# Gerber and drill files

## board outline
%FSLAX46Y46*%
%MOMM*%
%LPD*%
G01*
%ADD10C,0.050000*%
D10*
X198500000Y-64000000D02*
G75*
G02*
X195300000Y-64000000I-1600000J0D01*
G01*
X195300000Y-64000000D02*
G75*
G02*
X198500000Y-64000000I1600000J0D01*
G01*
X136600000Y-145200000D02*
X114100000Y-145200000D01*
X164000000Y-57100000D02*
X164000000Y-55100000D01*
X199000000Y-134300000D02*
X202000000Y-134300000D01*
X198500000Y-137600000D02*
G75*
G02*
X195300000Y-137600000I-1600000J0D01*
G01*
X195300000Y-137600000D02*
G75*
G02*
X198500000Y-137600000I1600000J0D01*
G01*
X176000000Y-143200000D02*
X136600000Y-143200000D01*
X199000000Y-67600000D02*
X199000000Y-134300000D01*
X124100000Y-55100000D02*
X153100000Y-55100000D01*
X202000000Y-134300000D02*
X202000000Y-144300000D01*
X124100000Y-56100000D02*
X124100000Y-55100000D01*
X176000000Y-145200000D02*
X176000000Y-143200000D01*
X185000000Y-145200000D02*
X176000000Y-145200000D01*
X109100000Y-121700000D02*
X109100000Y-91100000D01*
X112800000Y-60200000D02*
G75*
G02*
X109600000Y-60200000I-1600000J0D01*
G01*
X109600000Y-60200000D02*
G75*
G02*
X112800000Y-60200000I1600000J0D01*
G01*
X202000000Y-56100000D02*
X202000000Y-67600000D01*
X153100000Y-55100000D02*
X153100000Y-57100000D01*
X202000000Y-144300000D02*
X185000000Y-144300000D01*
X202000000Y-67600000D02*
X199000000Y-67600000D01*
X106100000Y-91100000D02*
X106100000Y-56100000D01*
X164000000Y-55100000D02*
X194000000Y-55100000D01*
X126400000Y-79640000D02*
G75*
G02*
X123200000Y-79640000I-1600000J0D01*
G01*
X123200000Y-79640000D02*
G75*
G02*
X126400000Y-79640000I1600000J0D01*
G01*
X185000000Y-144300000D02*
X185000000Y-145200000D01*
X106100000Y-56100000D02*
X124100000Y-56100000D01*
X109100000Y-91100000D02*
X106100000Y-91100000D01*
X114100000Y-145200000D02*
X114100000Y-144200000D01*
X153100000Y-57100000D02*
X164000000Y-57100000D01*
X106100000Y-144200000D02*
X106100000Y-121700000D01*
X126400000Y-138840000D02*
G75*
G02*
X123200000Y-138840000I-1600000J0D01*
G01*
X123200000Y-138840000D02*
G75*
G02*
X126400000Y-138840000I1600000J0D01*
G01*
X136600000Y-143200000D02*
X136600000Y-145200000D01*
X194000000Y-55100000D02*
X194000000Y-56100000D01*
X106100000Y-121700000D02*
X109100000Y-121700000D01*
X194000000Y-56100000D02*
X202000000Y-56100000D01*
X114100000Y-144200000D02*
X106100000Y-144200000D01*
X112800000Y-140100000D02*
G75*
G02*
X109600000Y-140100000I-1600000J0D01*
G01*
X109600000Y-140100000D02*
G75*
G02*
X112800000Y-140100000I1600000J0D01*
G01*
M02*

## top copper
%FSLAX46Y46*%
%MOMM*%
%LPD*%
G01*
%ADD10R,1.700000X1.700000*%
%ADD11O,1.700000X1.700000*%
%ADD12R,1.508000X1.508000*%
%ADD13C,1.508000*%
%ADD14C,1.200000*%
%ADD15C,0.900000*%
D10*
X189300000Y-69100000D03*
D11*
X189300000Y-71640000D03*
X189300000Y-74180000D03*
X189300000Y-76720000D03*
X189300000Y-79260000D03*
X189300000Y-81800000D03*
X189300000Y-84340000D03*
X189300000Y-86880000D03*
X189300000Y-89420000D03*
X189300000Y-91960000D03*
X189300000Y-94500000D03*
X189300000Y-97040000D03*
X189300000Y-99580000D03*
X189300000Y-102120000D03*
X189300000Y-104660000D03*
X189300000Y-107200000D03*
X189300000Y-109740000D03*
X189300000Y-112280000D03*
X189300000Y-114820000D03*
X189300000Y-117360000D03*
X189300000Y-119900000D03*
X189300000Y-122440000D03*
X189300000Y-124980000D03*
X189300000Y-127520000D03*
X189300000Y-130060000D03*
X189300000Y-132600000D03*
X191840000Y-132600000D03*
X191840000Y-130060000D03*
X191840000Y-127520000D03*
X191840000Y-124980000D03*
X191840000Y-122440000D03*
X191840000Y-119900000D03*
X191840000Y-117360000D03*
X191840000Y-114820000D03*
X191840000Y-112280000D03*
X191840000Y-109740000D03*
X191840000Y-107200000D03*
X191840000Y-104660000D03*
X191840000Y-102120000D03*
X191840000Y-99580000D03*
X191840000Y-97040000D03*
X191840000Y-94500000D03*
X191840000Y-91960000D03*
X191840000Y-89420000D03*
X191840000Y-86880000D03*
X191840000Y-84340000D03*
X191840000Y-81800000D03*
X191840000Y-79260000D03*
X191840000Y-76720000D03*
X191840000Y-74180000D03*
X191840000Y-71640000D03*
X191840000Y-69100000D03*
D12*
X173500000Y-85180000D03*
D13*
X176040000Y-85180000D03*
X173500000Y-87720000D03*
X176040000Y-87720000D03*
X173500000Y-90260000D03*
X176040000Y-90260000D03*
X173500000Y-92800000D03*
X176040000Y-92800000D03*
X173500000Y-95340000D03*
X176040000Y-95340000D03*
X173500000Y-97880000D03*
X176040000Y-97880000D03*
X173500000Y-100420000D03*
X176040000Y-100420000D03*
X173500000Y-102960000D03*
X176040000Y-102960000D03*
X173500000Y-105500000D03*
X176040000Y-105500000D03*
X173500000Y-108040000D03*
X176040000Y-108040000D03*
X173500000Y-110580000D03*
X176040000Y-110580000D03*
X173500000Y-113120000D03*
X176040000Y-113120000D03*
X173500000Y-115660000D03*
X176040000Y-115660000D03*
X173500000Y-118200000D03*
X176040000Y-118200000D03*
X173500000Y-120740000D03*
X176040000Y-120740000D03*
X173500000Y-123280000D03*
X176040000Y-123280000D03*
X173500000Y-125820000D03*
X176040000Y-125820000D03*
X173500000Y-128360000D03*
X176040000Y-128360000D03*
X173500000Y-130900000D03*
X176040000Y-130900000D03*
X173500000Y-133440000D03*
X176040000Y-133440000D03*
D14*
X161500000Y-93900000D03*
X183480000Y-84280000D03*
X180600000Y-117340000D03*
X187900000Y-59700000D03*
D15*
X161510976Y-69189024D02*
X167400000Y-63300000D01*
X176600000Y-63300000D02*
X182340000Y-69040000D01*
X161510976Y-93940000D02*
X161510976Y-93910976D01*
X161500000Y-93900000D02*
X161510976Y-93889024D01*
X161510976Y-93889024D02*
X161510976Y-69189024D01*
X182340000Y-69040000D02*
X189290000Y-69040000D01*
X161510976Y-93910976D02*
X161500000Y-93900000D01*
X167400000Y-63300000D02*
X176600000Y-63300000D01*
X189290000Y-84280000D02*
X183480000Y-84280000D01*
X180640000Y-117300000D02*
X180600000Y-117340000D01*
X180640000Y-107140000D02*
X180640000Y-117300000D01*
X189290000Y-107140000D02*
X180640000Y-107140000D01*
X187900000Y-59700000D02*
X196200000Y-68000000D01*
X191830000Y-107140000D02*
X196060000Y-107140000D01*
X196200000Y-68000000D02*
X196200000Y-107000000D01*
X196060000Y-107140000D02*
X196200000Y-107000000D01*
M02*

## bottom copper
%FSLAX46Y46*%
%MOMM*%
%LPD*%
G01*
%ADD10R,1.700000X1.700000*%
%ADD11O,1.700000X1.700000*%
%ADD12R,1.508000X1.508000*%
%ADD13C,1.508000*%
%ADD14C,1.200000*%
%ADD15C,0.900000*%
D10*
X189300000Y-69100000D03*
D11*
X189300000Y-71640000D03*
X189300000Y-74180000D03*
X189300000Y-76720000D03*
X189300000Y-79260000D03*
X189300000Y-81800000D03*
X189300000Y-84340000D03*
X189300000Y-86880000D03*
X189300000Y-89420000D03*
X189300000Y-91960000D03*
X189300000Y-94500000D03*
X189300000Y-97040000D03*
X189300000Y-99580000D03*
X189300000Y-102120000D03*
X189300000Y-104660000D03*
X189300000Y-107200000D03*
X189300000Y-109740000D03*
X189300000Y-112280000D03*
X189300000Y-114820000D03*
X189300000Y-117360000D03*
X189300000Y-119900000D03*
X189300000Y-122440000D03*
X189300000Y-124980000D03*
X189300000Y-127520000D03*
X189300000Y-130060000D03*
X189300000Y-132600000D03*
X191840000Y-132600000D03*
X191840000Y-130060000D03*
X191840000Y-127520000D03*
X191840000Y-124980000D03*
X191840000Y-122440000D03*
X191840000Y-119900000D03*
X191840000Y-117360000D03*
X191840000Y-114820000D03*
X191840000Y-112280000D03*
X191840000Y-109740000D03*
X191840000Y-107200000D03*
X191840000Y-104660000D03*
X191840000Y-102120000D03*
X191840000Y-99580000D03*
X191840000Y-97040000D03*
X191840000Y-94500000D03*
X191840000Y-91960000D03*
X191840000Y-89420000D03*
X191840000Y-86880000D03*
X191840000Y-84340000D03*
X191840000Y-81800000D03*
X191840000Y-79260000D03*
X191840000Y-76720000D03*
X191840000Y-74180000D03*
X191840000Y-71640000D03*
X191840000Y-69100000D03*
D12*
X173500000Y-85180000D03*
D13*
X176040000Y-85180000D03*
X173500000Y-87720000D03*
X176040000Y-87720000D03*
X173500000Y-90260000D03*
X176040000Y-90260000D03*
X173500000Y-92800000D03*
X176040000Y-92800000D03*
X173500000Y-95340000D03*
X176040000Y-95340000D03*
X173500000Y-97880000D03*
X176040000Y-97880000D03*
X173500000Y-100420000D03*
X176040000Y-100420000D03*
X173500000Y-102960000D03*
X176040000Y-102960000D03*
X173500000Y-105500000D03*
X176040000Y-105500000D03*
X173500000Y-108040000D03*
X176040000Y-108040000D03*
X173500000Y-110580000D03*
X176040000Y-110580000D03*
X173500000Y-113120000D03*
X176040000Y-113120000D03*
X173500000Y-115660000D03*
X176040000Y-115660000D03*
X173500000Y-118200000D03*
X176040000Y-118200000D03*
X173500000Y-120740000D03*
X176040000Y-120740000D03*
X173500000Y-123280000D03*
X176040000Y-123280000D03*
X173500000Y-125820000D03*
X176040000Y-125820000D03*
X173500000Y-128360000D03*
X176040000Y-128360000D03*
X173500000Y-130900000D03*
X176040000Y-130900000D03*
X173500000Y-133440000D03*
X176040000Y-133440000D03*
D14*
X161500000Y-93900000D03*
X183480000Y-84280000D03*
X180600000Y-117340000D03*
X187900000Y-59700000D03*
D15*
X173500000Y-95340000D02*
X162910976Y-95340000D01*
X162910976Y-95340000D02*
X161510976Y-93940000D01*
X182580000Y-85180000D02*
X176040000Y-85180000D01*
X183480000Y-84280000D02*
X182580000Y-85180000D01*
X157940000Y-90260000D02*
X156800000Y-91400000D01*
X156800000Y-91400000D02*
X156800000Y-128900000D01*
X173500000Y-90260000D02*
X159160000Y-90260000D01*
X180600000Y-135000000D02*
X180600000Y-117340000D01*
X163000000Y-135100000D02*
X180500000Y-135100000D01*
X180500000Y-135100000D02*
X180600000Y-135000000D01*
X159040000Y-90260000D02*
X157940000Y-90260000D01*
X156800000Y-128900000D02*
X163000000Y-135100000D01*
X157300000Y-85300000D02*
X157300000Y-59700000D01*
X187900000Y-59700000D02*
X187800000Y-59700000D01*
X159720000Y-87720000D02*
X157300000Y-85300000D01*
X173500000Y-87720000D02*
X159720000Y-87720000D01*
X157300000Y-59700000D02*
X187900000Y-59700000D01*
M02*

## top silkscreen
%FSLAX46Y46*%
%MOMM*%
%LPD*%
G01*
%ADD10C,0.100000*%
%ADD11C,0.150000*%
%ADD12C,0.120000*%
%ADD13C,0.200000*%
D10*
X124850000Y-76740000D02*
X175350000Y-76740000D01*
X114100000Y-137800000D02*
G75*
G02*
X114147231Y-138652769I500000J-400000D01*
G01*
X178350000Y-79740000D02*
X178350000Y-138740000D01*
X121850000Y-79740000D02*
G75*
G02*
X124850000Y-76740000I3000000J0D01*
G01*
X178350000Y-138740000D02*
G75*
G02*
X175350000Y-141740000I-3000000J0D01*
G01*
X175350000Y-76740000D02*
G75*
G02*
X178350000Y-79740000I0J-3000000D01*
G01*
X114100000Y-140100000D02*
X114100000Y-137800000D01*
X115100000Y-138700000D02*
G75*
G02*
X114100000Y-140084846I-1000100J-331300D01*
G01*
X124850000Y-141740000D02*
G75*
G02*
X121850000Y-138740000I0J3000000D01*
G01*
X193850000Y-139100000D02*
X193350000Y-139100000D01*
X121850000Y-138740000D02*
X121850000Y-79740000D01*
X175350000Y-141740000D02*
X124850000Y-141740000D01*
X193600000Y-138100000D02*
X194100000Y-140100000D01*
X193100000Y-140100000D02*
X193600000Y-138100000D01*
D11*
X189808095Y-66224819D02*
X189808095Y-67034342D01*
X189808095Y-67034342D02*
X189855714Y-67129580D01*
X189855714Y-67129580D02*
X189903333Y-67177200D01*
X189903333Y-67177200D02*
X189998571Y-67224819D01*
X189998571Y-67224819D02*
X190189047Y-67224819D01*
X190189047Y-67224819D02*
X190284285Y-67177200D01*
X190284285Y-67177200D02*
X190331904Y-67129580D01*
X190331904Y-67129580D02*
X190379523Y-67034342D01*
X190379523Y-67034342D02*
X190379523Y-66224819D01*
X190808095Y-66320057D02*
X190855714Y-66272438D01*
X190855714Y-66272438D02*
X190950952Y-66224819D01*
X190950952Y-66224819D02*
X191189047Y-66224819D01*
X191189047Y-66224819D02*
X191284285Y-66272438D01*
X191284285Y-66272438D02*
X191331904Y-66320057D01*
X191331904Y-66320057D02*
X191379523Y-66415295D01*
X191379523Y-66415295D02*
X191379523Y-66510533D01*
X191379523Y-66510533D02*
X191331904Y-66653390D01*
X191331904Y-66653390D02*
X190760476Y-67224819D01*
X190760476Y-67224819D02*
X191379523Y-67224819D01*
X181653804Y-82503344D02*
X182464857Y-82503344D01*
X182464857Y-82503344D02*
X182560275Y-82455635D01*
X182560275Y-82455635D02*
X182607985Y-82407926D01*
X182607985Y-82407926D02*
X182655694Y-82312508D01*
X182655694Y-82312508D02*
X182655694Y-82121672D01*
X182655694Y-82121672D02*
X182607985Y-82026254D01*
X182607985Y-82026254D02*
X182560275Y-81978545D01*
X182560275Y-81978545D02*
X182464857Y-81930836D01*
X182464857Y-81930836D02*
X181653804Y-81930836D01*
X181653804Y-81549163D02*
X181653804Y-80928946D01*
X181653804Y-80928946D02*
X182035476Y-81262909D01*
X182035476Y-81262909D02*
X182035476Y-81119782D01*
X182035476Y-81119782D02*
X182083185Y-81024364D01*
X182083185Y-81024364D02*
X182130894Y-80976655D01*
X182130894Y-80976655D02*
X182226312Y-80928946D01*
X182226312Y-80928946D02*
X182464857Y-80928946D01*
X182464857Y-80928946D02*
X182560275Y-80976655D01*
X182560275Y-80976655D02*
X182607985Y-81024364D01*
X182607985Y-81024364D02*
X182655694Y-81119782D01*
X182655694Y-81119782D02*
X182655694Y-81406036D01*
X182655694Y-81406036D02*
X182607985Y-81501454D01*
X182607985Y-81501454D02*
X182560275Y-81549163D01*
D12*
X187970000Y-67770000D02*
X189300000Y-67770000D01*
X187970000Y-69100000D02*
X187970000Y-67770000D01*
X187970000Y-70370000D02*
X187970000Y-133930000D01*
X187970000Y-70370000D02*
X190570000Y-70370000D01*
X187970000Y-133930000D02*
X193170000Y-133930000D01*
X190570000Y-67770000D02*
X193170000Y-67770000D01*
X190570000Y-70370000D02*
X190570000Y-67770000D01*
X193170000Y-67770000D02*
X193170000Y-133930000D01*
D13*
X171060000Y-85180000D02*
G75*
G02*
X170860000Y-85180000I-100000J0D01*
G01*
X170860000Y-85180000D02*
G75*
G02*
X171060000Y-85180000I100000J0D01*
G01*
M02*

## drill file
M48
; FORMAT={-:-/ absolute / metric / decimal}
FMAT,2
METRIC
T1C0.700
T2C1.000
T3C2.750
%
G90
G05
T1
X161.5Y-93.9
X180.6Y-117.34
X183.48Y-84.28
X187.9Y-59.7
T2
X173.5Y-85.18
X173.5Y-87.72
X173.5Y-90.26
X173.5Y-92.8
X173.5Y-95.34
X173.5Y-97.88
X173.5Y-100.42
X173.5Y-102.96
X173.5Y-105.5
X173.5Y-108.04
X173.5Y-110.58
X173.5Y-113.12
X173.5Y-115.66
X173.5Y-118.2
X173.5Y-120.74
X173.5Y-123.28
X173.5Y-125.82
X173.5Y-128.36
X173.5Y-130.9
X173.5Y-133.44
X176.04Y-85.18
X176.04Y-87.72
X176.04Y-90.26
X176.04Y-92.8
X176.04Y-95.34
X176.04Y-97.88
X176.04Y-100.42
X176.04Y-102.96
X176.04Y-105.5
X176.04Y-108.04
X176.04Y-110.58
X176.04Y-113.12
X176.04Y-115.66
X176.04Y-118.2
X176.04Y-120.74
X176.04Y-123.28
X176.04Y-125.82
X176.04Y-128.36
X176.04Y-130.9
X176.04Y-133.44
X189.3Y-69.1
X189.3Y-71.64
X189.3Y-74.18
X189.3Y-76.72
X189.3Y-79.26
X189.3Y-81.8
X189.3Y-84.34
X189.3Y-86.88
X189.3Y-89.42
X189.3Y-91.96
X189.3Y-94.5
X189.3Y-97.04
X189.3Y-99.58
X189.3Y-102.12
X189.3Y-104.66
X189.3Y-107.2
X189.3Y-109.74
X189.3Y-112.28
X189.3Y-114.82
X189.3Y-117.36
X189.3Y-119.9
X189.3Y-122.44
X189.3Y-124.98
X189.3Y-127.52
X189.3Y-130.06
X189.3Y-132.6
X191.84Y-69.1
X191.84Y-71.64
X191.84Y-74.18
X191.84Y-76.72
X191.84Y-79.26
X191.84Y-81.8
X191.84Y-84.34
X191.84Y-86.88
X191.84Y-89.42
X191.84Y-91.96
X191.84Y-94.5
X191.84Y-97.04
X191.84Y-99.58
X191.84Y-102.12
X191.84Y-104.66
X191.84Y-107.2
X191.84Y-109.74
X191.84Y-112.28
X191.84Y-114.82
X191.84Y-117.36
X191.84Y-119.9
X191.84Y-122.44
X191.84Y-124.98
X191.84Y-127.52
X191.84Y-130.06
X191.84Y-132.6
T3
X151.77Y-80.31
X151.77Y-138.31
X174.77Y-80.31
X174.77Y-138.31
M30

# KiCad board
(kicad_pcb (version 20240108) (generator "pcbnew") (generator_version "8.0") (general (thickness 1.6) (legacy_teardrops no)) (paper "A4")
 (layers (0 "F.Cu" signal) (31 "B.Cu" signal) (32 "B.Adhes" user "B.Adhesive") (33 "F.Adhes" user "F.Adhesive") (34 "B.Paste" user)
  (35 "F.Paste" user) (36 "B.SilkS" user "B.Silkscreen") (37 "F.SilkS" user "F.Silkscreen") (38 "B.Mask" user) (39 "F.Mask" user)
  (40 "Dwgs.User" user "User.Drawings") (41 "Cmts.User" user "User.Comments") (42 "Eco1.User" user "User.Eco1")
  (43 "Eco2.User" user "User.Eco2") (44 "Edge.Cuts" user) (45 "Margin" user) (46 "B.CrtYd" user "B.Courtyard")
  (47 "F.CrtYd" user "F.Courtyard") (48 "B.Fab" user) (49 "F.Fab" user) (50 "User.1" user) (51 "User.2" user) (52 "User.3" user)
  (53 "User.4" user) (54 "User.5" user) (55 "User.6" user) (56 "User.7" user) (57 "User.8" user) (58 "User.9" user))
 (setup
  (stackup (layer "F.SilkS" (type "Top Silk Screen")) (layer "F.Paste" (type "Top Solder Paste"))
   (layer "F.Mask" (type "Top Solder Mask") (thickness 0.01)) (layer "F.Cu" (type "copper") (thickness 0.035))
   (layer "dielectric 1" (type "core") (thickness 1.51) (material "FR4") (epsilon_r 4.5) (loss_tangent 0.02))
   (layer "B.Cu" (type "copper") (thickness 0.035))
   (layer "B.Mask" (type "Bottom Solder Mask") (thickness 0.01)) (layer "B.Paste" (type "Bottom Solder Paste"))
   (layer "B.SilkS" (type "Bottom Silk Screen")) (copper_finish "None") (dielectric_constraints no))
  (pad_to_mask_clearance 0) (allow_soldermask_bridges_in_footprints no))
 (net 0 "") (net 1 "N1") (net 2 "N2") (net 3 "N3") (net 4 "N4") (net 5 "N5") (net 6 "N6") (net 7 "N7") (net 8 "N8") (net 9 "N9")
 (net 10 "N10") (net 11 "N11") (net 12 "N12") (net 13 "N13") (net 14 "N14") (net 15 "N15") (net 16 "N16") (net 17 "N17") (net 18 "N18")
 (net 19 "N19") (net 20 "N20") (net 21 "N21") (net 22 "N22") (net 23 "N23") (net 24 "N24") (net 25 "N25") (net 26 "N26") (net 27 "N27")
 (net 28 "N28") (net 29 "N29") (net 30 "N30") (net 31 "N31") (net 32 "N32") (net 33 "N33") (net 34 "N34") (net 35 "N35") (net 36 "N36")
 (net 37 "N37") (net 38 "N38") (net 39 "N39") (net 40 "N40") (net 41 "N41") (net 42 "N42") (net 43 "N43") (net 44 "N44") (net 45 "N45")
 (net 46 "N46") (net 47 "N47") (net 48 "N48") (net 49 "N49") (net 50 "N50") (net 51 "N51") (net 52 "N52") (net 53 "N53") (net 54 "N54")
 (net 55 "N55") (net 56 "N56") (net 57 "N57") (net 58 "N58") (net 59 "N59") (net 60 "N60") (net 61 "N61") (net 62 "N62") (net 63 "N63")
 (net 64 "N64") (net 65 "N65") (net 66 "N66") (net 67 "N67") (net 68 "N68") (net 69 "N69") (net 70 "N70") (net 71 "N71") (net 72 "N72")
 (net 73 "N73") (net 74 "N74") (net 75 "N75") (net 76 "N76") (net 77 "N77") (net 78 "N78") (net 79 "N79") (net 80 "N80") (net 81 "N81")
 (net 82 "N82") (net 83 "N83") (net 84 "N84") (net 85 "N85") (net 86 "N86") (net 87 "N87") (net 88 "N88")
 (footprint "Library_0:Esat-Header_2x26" (layer "F.Cu") (at 189.3 69.1)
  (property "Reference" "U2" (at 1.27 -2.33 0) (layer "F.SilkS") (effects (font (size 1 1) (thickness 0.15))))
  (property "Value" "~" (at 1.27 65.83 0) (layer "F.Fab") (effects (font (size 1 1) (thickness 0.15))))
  (fp_line (start -1.33 -1.33) (end 0 -1.33) (stroke (width 0.12) (type solid)) (layer "F.SilkS"))
  (fp_line (start -1.33 0) (end -1.33 -1.33) (stroke (width 0.12) (type solid)) (layer "F.SilkS"))
  (fp_line (start -1.33 1.27) (end -1.33 64.83) (stroke (width 0.12) (type solid)) (layer "F.SilkS"))
  (fp_line (start -1.33 1.27) (end 1.27 1.27) (stroke (width 0.12) (type solid)) (layer "F.SilkS"))
  (fp_line (start -1.33 64.83) (end 3.87 64.83) (stroke (width 0.12) (type solid)) (layer "F.SilkS"))
  (fp_line (start 1.27 -1.33) (end 3.87 -1.33) (stroke (width 0.12) (type solid)) (layer "F.SilkS"))
  (fp_line (start 1.27 1.27) (end 1.27 -1.33) (stroke (width 0.12) (type solid)) (layer "F.SilkS"))
  (fp_line (start 3.87 -1.33) (end 3.87 64.83) (stroke (width 0.12) (type solid)) (layer "F.SilkS"))
  (pad "1" thru_hole rect (at 0 0) (size 1.7 1.7) (drill 1) (layers "*.Cu" "*.Mask") (remove_unused_layers no) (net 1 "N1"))
  (pad "2" thru_hole oval (at 0 2.54) (size 1.7 1.7) (drill 1) (layers "*.Cu" "*.Mask" "B.Paste") (remove_unused_layers no) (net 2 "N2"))
  (pad "3" thru_hole oval (at 0 5.08) (size 1.7 1.7) (drill 1) (layers "*.Cu" "*.Mask") (remove_unused_layers no) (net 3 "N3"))
  (pad "4" thru_hole oval (at 0 7.62) (size 1.7 1.7) (drill 1) (layers "*.Cu" "*.Mask") (remove_unused_layers no) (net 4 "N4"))
  (pad "5" thru_hole oval (at 0 10.16) (size 1.7 1.7) (drill 1) (layers "*.Cu" "*.Mask") (remove_unused_layers no) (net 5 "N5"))
  (pad "6" thru_hole oval (at 0 12.7) (size 1.7 1.7) (drill 1) (layers "*.Cu" "*.Mask") (remove_unused_layers no) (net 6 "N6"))
  (pad "7" thru_hole oval (at 0 15.24) (size 1.7 1.7) (drill 1) (layers "*.Cu" "*.Mask") (remove_unused_layers no) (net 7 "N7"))
  (pad "8" thru_hole oval (at 0 17.78) (size 1.7 1.7) (drill 1) (layers "*.Cu" "*.Mask") (remove_unused_layers no) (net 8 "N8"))
  (pad "9" thru_hole oval (at 0 20.32) (size 1.7 1.7) (drill 1) (layers "*.Cu" "*.Mask") (remove_unused_layers no) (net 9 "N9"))
  (pad "10" thru_hole oval (at 0 22.86) (size 1.7 1.7) (drill 1) (layers "*.Cu" "*.Mask") (remove_unused_layers no) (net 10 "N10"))
  (pad "11" thru_hole oval (at 0 25.4) (size 1.7 1.7) (drill 1) (layers "*.Cu" "*.Mask") (remove_unused_layers no) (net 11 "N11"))
  (pad "12" thru_hole oval (at 0 27.94) (size 1.7 1.7) (drill 1) (layers "*.Cu" "*.Mask") (remove_unused_layers no) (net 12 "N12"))
  (pad "13" thru_hole oval (at 0 30.48) (size 1.7 1.7) (drill 1) (layers "*.Cu" "*.Mask") (remove_unused_layers no) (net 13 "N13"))
  (pad "14" thru_hole oval (at 0 33.02) (size 1.7 1.7) (drill 1) (layers "*.Cu" "*.Mask") (remove_unused_layers no) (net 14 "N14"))
  (pad "15" thru_hole oval (at 0 35.56) (size 1.7 1.7) (drill 1) (layers "*.Cu" "*.Mask") (remove_unused_layers no) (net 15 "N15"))
  (pad "16" thru_hole oval (at 0 38.1) (size 1.7 1.7) (drill 1) (layers "*.Cu" "*.Mask") (remove_unused_layers no) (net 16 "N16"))
  (pad "17" thru_hole oval (at 0 40.64) (size 1.7 1.7) (drill 1) (layers "*.Cu" "*.Mask") (remove_unused_layers no) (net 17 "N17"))
  (pad "18" thru_hole oval (at 0 43.18) (size 1.7 1.7) (drill 1) (layers "*.Cu" "*.Mask") (remove_unused_layers no) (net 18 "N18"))
  (pad "19" thru_hole oval (at 0 45.72) (size 1.7 1.7) (drill 1) (layers "*.Cu" "*.Mask") (remove_unused_layers no) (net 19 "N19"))
  (pad "20" thru_hole oval (at 0 48.26) (size 1.7 1.7) (drill 1) (layers "*.Cu" "*.Mask") (remove_unused_layers no) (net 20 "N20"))
  (pad "21" thru_hole oval (at 0 50.8) (size 1.7 1.7) (drill 1) (layers "*.Cu" "B.Mask") (remove_unused_layers no) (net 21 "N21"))
  (pad "22" thru_hole oval (at 0 53.34) (size 1.7 1.7) (drill 1) (layers "*.Cu" "*.Mask") (remove_unused_layers no) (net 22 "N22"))
  (pad "23" thru_hole oval (at 0 55.88) (size 1.7 1.7) (drill 1) (layers "*.Cu" "*.Mask") (remove_unused_layers no) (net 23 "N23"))
  (pad "24" thru_hole oval (at 0 58.42) (size 1.7 1.7) (drill 1) (layers "*.Cu" "*.Mask") (remove_unused_layers no) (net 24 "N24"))
  (pad "25" thru_hole oval (at 0 60.96) (size 1.7 1.7) (drill 1) (layers "*.Cu" "*.Mask") (remove_unused_layers no) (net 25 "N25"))
  (pad "26" thru_hole oval (at 0 63.5) (size 1.7 1.7) (drill 1) (layers "*.Cu" "*.Mask") (remove_unused_layers no) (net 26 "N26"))
  (pad "27" thru_hole oval (at 2.54 63.5) (size 1.7 1.7) (drill 1) (layers "*.Cu" "*.Mask") (remove_unused_layers no) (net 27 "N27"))
  (pad "28" thru_hole oval (at 2.54 60.96) (size 1.7 1.7) (drill 1) (layers "*.Cu" "*.Mask") (remove_unused_layers no) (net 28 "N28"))
  (pad "29" thru_hole oval (at 2.54 58.42) (size 1.7 1.7) (drill 1) (layers "*.Cu" "*.Mask") (remove_unused_layers no) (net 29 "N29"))
  (pad "30" thru_hole oval (at 2.54 55.88) (size 1.7 1.7) (drill 1) (layers "*.Cu" "*.Mask") (remove_unused_layers no) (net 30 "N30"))
  (pad "31" thru_hole oval (at 2.54 53.34) (size 1.7 1.7) (drill 1) (layers "*.Cu" "*.Mask") (remove_unused_layers no) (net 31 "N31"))
  (pad "32" thru_hole oval (at 2.54 50.8) (size 1.7 1.7) (drill 1) (layers "*.Cu" "*.Mask") (remove_unused_layers no) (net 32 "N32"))
  (pad "33" thru_hole oval (at 2.54 48.26) (size 1.7 1.7) (drill 1) (layers "*.Cu" "*.Mask") (remove_unused_layers no) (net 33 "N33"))
  (pad "34" thru_hole oval (at 2.54 45.72) (size 1.7 1.7) (drill 1) (layers "*.Cu" "*.Mask") (remove_unused_layers no) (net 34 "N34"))
  (pad "35" thru_hole oval (at 2.54 43.18) (size 1.7 1.7) (drill 1) (layers "*.Cu" "*.Mask") (remove_unused_layers no) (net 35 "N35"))
  (pad "36" thru_hole oval (at 2.54 40.64) (size 1.7 1.7) (drill 1) (layers "*.Cu" "*.Mask") (remove_unused_layers no) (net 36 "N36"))
  (pad "37" thru_hole oval (at 2.54 38.1) (size 1.7 1.7) (drill 1) (layers "*.Cu" "*.Mask") (remove_unused_layers no) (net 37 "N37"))
  (pad "38" thru_hole oval (at 2.54 35.56) (size 1.7 1.7) (drill 1) (layers "*.Cu" "*.Mask") (remove_unused_layers no) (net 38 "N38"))
  (pad "39" thru_hole oval (at 2.54 33.02) (size 1.7 1.7) (drill 1) (layers "*.Cu" "*.Mask" "B.Adhes") (remove_unused_layers no)
   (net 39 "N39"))
  (pad "40" thru_hole oval (at 2.54 30.48) (size 1.7 1.7) (drill 1) (layers "*.Cu" "*.Mask") (remove_unused_layers no) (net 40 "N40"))
  (pad "41" thru_hole oval (at 2.54 27.94) (size 1.7 1.7) (drill 1) (layers "*.Cu" "*.Mask") (remove_unused_layers no) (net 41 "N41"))
  (pad "42" thru_hole oval (at 2.54 25.4) (size 1.7 1.7) (drill 1) (layers "*.Cu" "*.Mask") (remove_unused_layers no) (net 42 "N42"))
  (pad "43" thru_hole oval (at 2.54 22.86) (size 1.7 1.7) (drill 1) (layers "*.Cu" "*.Mask") (remove_unused_layers no) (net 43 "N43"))
  (pad "44" thru_hole oval (at 2.54 20.32) (size 1.7 1.7) (drill 1) (layers "*.Cu" "*.Mask") (remove_unused_layers no) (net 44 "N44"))
  (pad "45" thru_hole oval (at 2.54 17.78) (size 1.7 1.7) (drill 1) (layers "*.Cu" "*.Mask") (remove_unused_layers no) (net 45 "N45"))
  (pad "46" thru_hole oval (at 2.54 15.24) (size 1.7 1.7) (drill 1) (layers "*.Cu" "*.Mask") (remove_unused_layers no) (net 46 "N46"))
  (pad "47" thru_hole oval (at 2.54 12.7) (size 1.7 1.7) (drill 1) (layers "*.Cu" "*.Mask") (remove_unused_layers no) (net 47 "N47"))
  (pad "48" thru_hole oval (at 2.54 10.16) (size 1.7 1.7) (drill 1) (layers "*.Cu" "*.Mask") (remove_unused_layers no) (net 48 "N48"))
  (pad "49" thru_hole oval (at 2.54 7.62) (size 1.7 1.7) (drill 1) (layers "*.Cu" "*.Mask") (remove_unused_layers no) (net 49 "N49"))
  (pad "50" thru_hole oval (at 2.54 5.08) (size 1.7 1.7) (drill 1) (layers "*.Cu" "*.Mask") (remove_unused_layers no) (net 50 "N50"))
  (pad "51" thru_hole oval (at 2.54 2.54) (size 1.7 1.7) (drill 1) (layers "*.Cu" "*.Mask") (remove_unused_layers no) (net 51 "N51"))
  (pad "52" thru_hole oval (at 2.54 0) (size 1.7 1.7) (drill 1) (layers "*.Cu" "*.Mask") (remove_unused_layers no) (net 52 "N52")))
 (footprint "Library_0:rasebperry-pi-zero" (layer "F.Cu") (at 163.27 109.31 -90)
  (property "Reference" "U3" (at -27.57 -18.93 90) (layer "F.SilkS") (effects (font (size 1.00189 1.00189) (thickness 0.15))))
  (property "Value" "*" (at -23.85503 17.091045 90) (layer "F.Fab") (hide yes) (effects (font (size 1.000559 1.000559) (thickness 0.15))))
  (fp_circle (center -24.13 -7.69) (end -24.03 -7.69) (stroke (width 0.2) (type solid)) (fill none) (layer "F.SilkS"))
  (pad "" np_thru_hole circle (at -29 -11.5 270) (size 2.75 2.75) (drill 2.75) (layers "*.Cu" "*.Mask"))
  (pad "" np_thru_hole circle (at -29 11.5 270) (size 2.75 2.75) (drill 2.75) (layers "*.Cu" "*.Mask"))
  (pad "" np_thru_hole circle (at 29 -11.5 270) (size 2.75 2.75) (drill 2.75) (layers "*.Cu" "*.Mask"))
  (pad "" np_thru_hole circle (at 29 11.5 270) (size 2.75 2.75) (drill 2.75) (layers "*.Cu" "*.Mask"))
  (pad "1" thru_hole rect (at -24.13 -10.23 270) (size 1.508 1.508) (drill 1) (layers "*.Cu" "*.Mask") (remove_unused_layers no)
   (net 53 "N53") (solder_mask_margin 0.102))
  (pad "2" thru_hole circle (at -24.13 -12.77 270) (size 1.508 1.508) (drill 1) (layers "*.Cu" "*.Mask") (remove_unused_layers no)
   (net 7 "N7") (solder_mask_margin 0.102))
  (pad "3" thru_hole circle (at -21.59 -10.23 270) (size 1.508 1.508) (drill 1) (layers "*.Cu" "*.Mask") (remove_unused_layers no)
   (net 37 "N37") (solder_mask_margin 0.102))
  (pad "4" thru_hole circle (at -21.59 -12.77 270) (size 1.508 1.508) (drill 1) (layers "*.Cu" "*.Mask") (remove_unused_layers no)
   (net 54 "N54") (solder_mask_margin 0.102))
  (pad "5" thru_hole circle (at -19.05 -10.23 270) (size 1.508 1.508) (drill 1) (layers "*.Cu" "*.Mask") (remove_unused_layers no)
   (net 16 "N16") (solder_mask_margin 0.102))
  (pad "6" thru_hole circle (at -19.05 -12.77 270) (size 1.508 1.508) (drill 1) (layers "*.Cu" "*.Mask") (remove_unused_layers no)
   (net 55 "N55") (solder_mask_margin 0.102))
  (pad "7" thru_hole circle (at -16.51 -10.23 270) (size 1.508 1.508) (drill 1) (layers "*.Cu" "*.Mask") (remove_unused_layers no)
   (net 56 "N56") (solder_mask_margin 0.102))
  (pad "8" thru_hole circle (at -16.51 -12.77 270) (size 1.508 1.508) (drill 1) (layers "*.Cu" "*.Mask") (remove_unused_layers no)
   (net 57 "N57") (solder_mask_margin 0.102))
  (pad "9" thru_hole circle (at -13.97 -10.23 270) (size 1.508 1.508) (drill 1) (layers "*.Cu" "*.Mask") (remove_unused_layers no)
   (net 1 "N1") (solder_mask_margin 0.102))
  (pad "10" thru_hole circle (at -13.97 -12.77 270) (size 1.508 1.508) (drill 1) (layers "*.Cu" "*.Mask") (remove_unused_layers no)
   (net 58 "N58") (solder_mask_margin 0.102))
  (pad "11" thru_hole circle (at -11.43 -10.23 270) (size 1.508 1.508) (drill 1) (layers "*.Cu" "*.Mask") (remove_unused_layers no)
   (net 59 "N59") (solder_mask_margin 0.102))
  (pad "12" thru_hole circle (at -11.43 -12.77 270) (size 1.508 1.508) (drill 1) (layers "*.Cu" "*.Mask") (remove_unused_layers no)
   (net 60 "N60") (solder_mask_margin 0.102))
  (pad "13" thru_hole circle (at -8.89 -10.23 270) (size 1.508 1.508) (drill 1) (layers "*.Cu" "*.Mask") (remove_unused_layers no)
   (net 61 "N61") (solder_mask_margin 0.102))
  (pad "14" thru_hole circle (at -8.89 -12.77 270) (size 1.508 1.508) (drill 1) (layers "*.Cu" "*.Mask") (remove_unused_layers no)
   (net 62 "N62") (solder_mask_margin 0.102))
  (pad "15" thru_hole circle (at -6.35 -10.23 270) (size 1.508 1.508) (drill 1) (layers "*.Cu" "*.Mask") (remove_unused_layers no)
   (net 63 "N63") (solder_mask_margin 0.102))
  (pad "16" thru_hole circle (at -6.35 -12.77 270) (size 1.508 1.508) (drill 1) (layers "*.Cu" "*.Mask") (remove_unused_layers no)
   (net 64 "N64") (solder_mask_margin 0.102))
  (pad "17" thru_hole circle (at -3.81 -10.23 270) (size 1.508 1.508) (drill 1) (layers "*.Cu" "*.Mask") (remove_unused_layers no)
   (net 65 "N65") (solder_mask_margin 0.102))
  (pad "18" thru_hole circle (at -3.81 -12.77 270) (size 1.508 1.508) (drill 1) (layers "*.Cu" "*.Mask") (remove_unused_layers no)
   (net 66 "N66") (solder_mask_margin 0.102))
  (pad "19" thru_hole circle (at -1.27 -10.23 270) (size 1.508 1.508) (drill 1) (layers "*.Cu" "*.Mask") (remove_unused_layers no)
   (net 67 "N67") (solder_mask_margin 0.102))
  (pad "20" thru_hole circle (at -1.27 -12.77 270) (size 1.508 1.508) (drill 1) (layers "*.Cu" "*.Mask") (remove_unused_layers no)
   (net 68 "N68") (solder_mask_margin 0.102))
  (pad "21" thru_hole circle (at 1.27 -10.23 270) (size 1.508 1.508) (drill 1) (layers "*.Cu" "*.Mask") (remove_unused_layers no)
   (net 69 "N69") (solder_mask_margin 0.102))
  (pad "22" thru_hole circle (at 1.27 -12.77 270) (size 1.508 1.508) (drill 1) (layers "*.Cu" "*.Mask") (remove_unused_layers no)
   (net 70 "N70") (solder_mask_margin 0.102))
  (pad "23" thru_hole circle (at 3.81 -10.23 270) (size 1.508 1.508) (drill 1) (layers "*.Cu" "*.Mask") (remove_unused_layers no)
   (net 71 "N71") (solder_mask_margin 0.102))
  (pad "24" thru_hole circle (at 3.81 -12.77 270) (size 1.508 1.508) (drill 1) (layers "*.Cu" "*.Mask") (remove_unused_layers no)
   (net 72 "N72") (solder_mask_margin 0.102))
  (pad "25" thru_hole circle (at 6.35 -10.23 270) (size 1.508 1.508) (drill 1) (layers "*.Cu" "*.Mask") (remove_unused_layers no)
   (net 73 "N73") (solder_mask_margin 0.102))
  (pad "26" thru_hole circle (at 6.35 -12.77 270) (size 1.508 1.508) (drill 1) (layers "*.Cu" "*.Mask") (remove_unused_layers no)
   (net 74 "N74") (solder_mask_margin 0.102))
  (pad "27" thru_hole circle (at 8.89 -10.23 270) (size 1.508 1.508) (drill 1) (layers "*.Cu" "*.Mask") (remove_unused_layers no)
   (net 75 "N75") (solder_mask_margin 0.102))
  (pad "28" thru_hole circle (at 8.89 -12.77 270) (size 1.508 1.508) (drill 1) (layers "*.Cu" "*.Mask") (remove_unused_layers no)
   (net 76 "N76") (solder_mask_margin 0.102))
  (pad "29" thru_hole circle (at 11.43 -10.23 270) (size 1.508 1.508) (drill 1) (layers "*.Cu" "*.Mask") (remove_unused_layers no)
   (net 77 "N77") (solder_mask_margin 0.102))
  (pad "30" thru_hole circle (at 11.43 -12.77 270) (size 1.508 1.508) (drill 1) (layers "*.Cu" "*.Mask") (remove_unused_layers no)
   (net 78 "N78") (solder_mask_margin 0.102))
  (pad "31" thru_hole circle (at 13.97 -10.23 270) (size 1.508 1.508) (drill 1) (layers "*.Cu" "*.Mask") (remove_unused_layers no)
   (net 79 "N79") (solder_mask_margin 0.102))
  (pad "32" thru_hole circle (at 13.97 -12.77 270) (size 1.508 1.508) (drill 1) (layers "*.Cu" "*.Mask") (remove_unused_layers no)
   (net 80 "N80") (solder_mask_margin 0.102))
  (pad "33" thru_hole circle (at 16.51 -10.23 270) (size 1.508 1.508) (drill 1) (layers "*.Cu" "*.Mask") (remove_unused_layers no)
   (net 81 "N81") (solder_mask_margin 0.102))
  (pad "34" thru_hole circle (at 16.51 -12.77 270) (size 1.508 1.508) (drill 1) (layers "*.Cu" "*.Mask") (remove_unused_layers no)
   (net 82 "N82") (solder_mask_margin 0.102))
  (pad "35" thru_hole circle (at 19.05 -10.23 270) (size 1.508 1.508) (drill 1) (layers "*.Cu" "*.Mask") (remove_unused_layers no)
   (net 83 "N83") (solder_mask_margin 0.102))
  (pad "36" thru_hole circle (at 19.05 -12.77 270) (size 1.508 1.508) (drill 1) (layers "*.Cu" "*.Mask") (remove_unused_layers no)
   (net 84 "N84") (solder_mask_margin 0.102))
  (pad "37" thru_hole circle (at 21.59 -10.23 270) (size 1.508 1.508) (drill 1) (layers "*.Cu" "*.Mask") (remove_unused_layers no)
   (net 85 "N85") (solder_mask_margin 0.102))
  (pad "38" thru_hole circle (at 21.59 -12.77 270) (size 1.508 1.508) (drill 1) (layers "*.Cu" "*.Mask") (remove_unused_layers no)
   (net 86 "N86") (solder_mask_margin 0.102))
  (pad "39" thru_hole circle (at 24.13 -10.23 270) (size 1.508 1.508) (drill 1) (layers "*.Cu" "*.Mask") (remove_unused_layers no)
   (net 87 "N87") (solder_mask_margin 0.102))
  (pad "40" thru_hole circle (at 24.13 -12.77 270) (size 1.508 1.508) (drill 1) (layers "*.Cu" "*.Mask") (remove_unused_layers no)
   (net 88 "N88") (solder_mask_margin 0.102)))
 (gr_line (start 124.85 76.74) (end 175.35 76.74) (stroke (width 0.1) (type default)) (layer "F.SilkS"))
 (gr_arc (start 114.1 137.8) (mid 115.239333 138.16459) (end 114.147231 138.652769) (stroke (width 0.1) (type default)) (layer "F.SilkS"))
 (gr_line (start 178.35 79.74) (end 178.35 138.74) (stroke (width 0.1) (type default)) (layer "F.SilkS"))
 (gr_arc (start 121.85 79.74) (mid 122.72868 77.61868) (end 124.85 76.74) (stroke (width 0.1) (type default)) (layer "F.SilkS"))
 (gr_arc (start 178.35 138.74) (mid 177.47132 140.86132) (end 175.35 141.74) (stroke (width 0.1) (type default)) (layer "F.SilkS"))
 (gr_arc (start 175.35 76.74) (mid 177.47132 77.61868) (end 178.35 79.74) (stroke (width 0.1) (type default)) (layer "F.SilkS"))
 (gr_line (start 114.1 140.1) (end 114.1 137.8) (stroke (width 0.1) (type default)) (layer "F.SilkS"))
 (gr_arc (start 115.1 138.7) (mid 114.954033 139.648055) (end 114.1 140.084797) (stroke (width 0.1) (type default)) (layer "F.SilkS"))
 (gr_arc (start 124.85 141.74) (mid 122.72868 140.86132) (end 121.85 138.74) (stroke (width 0.1) (type default)) (layer "F.SilkS"))
 (gr_line (start 193.85 139.1) (end 193.35 139.1) (stroke (width 0.1) (type default)) (layer "F.SilkS"))
 (gr_line (start 121.85 138.74) (end 121.85 79.74) (stroke (width 0.1) (type default)) (layer "F.SilkS"))
 (gr_line (start 175.35 141.74) (end 124.85 141.74) (stroke (width 0.1) (type default)) (layer "F.SilkS"))
 (gr_line (start 193.6 138.1) (end 194.1 140.1) (stroke (width 0.1) (type default)) (layer "F.SilkS"))
 (gr_line (start 193.1 140.1) (end 193.6 138.1) (stroke (width 0.1) (type default)) (layer "F.SilkS"))
 (gr_circle (center 196.9 64) (end 196.9 65.6) (stroke (width 0.05) (type default)) (fill none) (layer "Edge.Cuts"))
 (gr_line (start 136.6 145.2) (end 114.1 145.2) (stroke (width 0.05) (type default)) (layer "Edge.Cuts"))
 (gr_line (start 164 57.1) (end 164 55.1) (stroke (width 0.05) (type default)) (layer "Edge.Cuts"))
 (gr_line (start 199 134.3) (end 202 134.3) (stroke (width 0.05) (type default)) (layer "Edge.Cuts"))
 (gr_circle (center 196.9 137.6) (end 196.9 139.2) (stroke (width 0.05) (type default)) (fill none) (layer "Edge.Cuts"))
 (gr_line (start 176 143.2) (end 136.6 143.2) (stroke (width 0.05) (type default)) (layer "Edge.Cuts"))
 (gr_line (start 199 67.6) (end 199 134.3) (stroke (width 0.05) (type default)) (layer "Edge.Cuts"))
 (gr_line (start 124.1 55.1) (end 153.1 55.1) (stroke (width 0.05) (type default)) (layer "Edge.Cuts"))
 (gr_line (start 202 134.3) (end 202 144.3) (stroke (width 0.05) (type default)) (layer "Edge.Cuts"))
 (gr_line (start 124.1 56.1) (end 124.1 55.1) (stroke (width 0.05) (type default)) (layer "Edge.Cuts"))
 (gr_line (start 176 145.2) (end 176 143.2) (stroke (width 0.05) (type default)) (layer "Edge.Cuts"))
 (gr_line (start 185 145.2) (end 176 145.2) (stroke (width 0.05) (type default)) (layer "Edge.Cuts"))
 (gr_line (start 109.1 121.7) (end 109.1 91.1) (stroke (width 0.05) (type default)) (layer "Edge.Cuts"))
 (gr_circle (center 111.2 60.2) (end 111.2 61.8) (stroke (width 0.05) (type default)) (fill none) (layer "Edge.Cuts"))
 (gr_line (start 202 56.1) (end 202 67.6) (stroke (width 0.05) (type default)) (layer "Edge.Cuts"))
 (gr_line (start 153.1 55.1) (end 153.1 57.1) (stroke (width 0.05) (type default)) (layer "Edge.Cuts"))
 (gr_line (start 202 144.3) (end 185 144.3) (stroke (width 0.05) (type default)) (layer "Edge.Cuts"))
 (gr_line (start 202 67.6) (end 199 67.6) (stroke (width 0.05) (type default)) (layer "Edge.Cuts"))
 (gr_line (start 106.1 91.1) (end 106.1 56.1) (stroke (width 0.05) (type default)) (layer "Edge.Cuts"))
 (gr_line (start 164 55.1) (end 194 55.1) (stroke (width 0.05) (type default)) (layer "Edge.Cuts"))
 (gr_circle (center 124.8 79.64) (end 124.8 81.24) (stroke (width 0.05) (type default)) (fill none) (layer "Edge.Cuts"))
 (gr_line (start 185 144.3) (end 185 145.2) (stroke (width 0.05) (type default)) (layer "Edge.Cuts"))
 (gr_line (start 106.1 56.1) (end 124.1 56.1) (stroke (width 0.05) (type default)) (layer "Edge.Cuts"))
 (gr_line (start 109.1 91.1) (end 106.1 91.1) (stroke (width 0.05) (type default)) (layer "Edge.Cuts"))
 (gr_line (start 114.1 145.2) (end 114.1 144.2) (stroke (width 0.05) (type default)) (layer "Edge.Cuts"))
 (gr_line (start 153.1 57.1) (end 164 57.1) (stroke (width 0.05) (type default)) (layer "Edge.Cuts"))
 (gr_line (start 106.1 144.2) (end 106.1 121.7) (stroke (width 0.05) (type default)) (layer "Edge.Cuts"))
 (gr_circle (center 124.8 138.84) (end 124.8 140.44) (stroke (width 0.05) (type default)) (fill none) (layer "Edge.Cuts"))
 (gr_line (start 136.6 143.2) (end 136.6 145.2) (stroke (width 0.05) (type default)) (layer "Edge.Cuts"))
 (gr_line (start 194 55.1) (end 194 56.1) (stroke (width 0.05) (type default)) (layer "Edge.Cuts"))
 (gr_line (start 106.1 121.7) (end 109.1 121.7) (stroke (width 0.05) (type default)) (layer "Edge.Cuts"))
 (gr_line (start 194 56.1) (end 202 56.1) (stroke (width 0.05) (type default)) (layer "Edge.Cuts"))
 (gr_line (start 114.1 144.2) (end 106.1 144.2) (stroke (width 0.05) (type default)) (layer "Edge.Cuts"))
 (gr_circle (center 111.2 140.1) (end 111.2 141.7) (stroke (width 0.05) (type default)) (fill none) (layer "Edge.Cuts"))
 (segment (start 161.510976 69.189024) (end 167.4 63.3) (width 0.9) (layer "F.Cu") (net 1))
 (segment (start 176.6 63.3) (end 182.34 69.04) (width 0.9) (layer "F.Cu") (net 1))
 (segment (start 161.510976 93.94) (end 161.510976 93.910976) (width 0.9) (layer "F.Cu") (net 1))
 (segment (start 161.5 93.9) (end 161.510976 93.889024) (width 0.9) (layer "F.Cu") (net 1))
 (segment (start 161.510976 93.889024) (end 161.510976 69.189024) (width 0.9) (layer "F.Cu") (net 1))
 (segment (start 182.34 69.04) (end 189.29 69.04) (width 0.9) (layer "F.Cu") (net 1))
 (segment (start 161.510976 93.910976) (end 161.5 93.9) (width 0.9) (layer "F.Cu") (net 1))
 (segment (start 167.4 63.3) (end 176.6 63.3) (width 0.9) (layer "F.Cu") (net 1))
 (via (at 161.5 93.9) (size 1.2) (drill 0.7) (layers "F.Cu" "B.Cu") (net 1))
 (segment (start 173.5 95.34) (end 162.910976 95.34) (width 0.9) (layer "B.Cu") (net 1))
 (segment (start 162.910976 95.34) (end 161.510976 93.94) (width 0.9) (layer "B.Cu") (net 1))
 (segment (start 189.29 84.28) (end 183.48 84.28) (width 0.9) (layer "F.Cu") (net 7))
 (via (at 183.48 84.28) (size 1.2) (drill 0.7) (layers "F.Cu" "B.Cu") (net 7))
 (segment (start 182.58 85.18) (end 176.04 85.18) (width 0.9) (layer "B.Cu") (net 7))
 (segment (start 183.48 84.28) (end 182.58 85.18) (width 0.9) (layer "B.Cu") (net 7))
 (segment (start 180.64 117.3) (end 180.6 117.34) (width 0.9) (layer "F.Cu") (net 16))
 (segment (start 180.64 107.14) (end 180.64 117.3) (width 0.9) (layer "F.Cu") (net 16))
 (segment (start 189.29 107.14) (end 180.64 107.14) (width 0.9) (layer "F.Cu") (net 16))
 (via (at 180.6 117.34) (size 1.2) (drill 0.7) (layers "F.Cu" "B.Cu") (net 16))
 (segment (start 157.94 90.26) (end 156.8 91.4) (width 0.9) (layer "B.Cu") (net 16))
 (segment (start 156.8 91.4) (end 156.8 128.9) (width 0.9) (layer "B.Cu") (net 16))
 (segment (start 173.5 90.26) (end 159.16 90.26) (width 0.9) (layer "B.Cu") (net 16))
 (segment (start 180.6 135) (end 180.6 117.34) (width 0.9) (layer "B.Cu") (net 16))
 (segment (start 163 135.1) (end 180.5 135.1) (width 0.9) (layer "B.Cu") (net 16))
 (segment (start 180.5 135.1) (end 180.6 135) (width 0.9) (layer "B.Cu") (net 16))
 (segment (start 159.04 90.26) (end 157.94 90.26) (width 0.9) (layer "B.Cu") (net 16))
 (segment (start 156.8 128.9) (end 163 135.1) (width 0.9) (layer "B.Cu") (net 16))
 (segment (start 187.9 59.7) (end 196.2 68) (width 0.9) (layer "F.Cu") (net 37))
 (segment (start 191.83 107.14) (end 196.06 107.14) (width 0.9) (layer "F.Cu") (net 37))
 (segment (start 196.2 68) (end 196.2 107) (width 0.9) (layer "F.Cu") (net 37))
 (segment (start 196.06 107.14) (end 196.2 107) (width 0.9) (layer "F.Cu") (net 37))
 (via (at 187.9 59.7) (size 1.2) (drill 0.7) (layers "F.Cu" "B.Cu") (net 37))
 (segment (start 157.3 85.3) (end 157.3 59.7) (width 0.9) (layer "B.Cu") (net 37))
 (segment (start 187.9 59.7) (end 187.8 59.7) (width 0.9) (layer "B.Cu") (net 37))
 (segment (start 159.72 87.72) (end 157.3 85.3) (width 0.9) (layer "B.Cu") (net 37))
 (segment (start 173.5 87.72) (end 159.72 87.72) (width 0.9) (layer "B.Cu") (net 37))
 (segment (start 157.3 59.7) (end 187.9 59.7) (width 0.9) (layer "B.Cu") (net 37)))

